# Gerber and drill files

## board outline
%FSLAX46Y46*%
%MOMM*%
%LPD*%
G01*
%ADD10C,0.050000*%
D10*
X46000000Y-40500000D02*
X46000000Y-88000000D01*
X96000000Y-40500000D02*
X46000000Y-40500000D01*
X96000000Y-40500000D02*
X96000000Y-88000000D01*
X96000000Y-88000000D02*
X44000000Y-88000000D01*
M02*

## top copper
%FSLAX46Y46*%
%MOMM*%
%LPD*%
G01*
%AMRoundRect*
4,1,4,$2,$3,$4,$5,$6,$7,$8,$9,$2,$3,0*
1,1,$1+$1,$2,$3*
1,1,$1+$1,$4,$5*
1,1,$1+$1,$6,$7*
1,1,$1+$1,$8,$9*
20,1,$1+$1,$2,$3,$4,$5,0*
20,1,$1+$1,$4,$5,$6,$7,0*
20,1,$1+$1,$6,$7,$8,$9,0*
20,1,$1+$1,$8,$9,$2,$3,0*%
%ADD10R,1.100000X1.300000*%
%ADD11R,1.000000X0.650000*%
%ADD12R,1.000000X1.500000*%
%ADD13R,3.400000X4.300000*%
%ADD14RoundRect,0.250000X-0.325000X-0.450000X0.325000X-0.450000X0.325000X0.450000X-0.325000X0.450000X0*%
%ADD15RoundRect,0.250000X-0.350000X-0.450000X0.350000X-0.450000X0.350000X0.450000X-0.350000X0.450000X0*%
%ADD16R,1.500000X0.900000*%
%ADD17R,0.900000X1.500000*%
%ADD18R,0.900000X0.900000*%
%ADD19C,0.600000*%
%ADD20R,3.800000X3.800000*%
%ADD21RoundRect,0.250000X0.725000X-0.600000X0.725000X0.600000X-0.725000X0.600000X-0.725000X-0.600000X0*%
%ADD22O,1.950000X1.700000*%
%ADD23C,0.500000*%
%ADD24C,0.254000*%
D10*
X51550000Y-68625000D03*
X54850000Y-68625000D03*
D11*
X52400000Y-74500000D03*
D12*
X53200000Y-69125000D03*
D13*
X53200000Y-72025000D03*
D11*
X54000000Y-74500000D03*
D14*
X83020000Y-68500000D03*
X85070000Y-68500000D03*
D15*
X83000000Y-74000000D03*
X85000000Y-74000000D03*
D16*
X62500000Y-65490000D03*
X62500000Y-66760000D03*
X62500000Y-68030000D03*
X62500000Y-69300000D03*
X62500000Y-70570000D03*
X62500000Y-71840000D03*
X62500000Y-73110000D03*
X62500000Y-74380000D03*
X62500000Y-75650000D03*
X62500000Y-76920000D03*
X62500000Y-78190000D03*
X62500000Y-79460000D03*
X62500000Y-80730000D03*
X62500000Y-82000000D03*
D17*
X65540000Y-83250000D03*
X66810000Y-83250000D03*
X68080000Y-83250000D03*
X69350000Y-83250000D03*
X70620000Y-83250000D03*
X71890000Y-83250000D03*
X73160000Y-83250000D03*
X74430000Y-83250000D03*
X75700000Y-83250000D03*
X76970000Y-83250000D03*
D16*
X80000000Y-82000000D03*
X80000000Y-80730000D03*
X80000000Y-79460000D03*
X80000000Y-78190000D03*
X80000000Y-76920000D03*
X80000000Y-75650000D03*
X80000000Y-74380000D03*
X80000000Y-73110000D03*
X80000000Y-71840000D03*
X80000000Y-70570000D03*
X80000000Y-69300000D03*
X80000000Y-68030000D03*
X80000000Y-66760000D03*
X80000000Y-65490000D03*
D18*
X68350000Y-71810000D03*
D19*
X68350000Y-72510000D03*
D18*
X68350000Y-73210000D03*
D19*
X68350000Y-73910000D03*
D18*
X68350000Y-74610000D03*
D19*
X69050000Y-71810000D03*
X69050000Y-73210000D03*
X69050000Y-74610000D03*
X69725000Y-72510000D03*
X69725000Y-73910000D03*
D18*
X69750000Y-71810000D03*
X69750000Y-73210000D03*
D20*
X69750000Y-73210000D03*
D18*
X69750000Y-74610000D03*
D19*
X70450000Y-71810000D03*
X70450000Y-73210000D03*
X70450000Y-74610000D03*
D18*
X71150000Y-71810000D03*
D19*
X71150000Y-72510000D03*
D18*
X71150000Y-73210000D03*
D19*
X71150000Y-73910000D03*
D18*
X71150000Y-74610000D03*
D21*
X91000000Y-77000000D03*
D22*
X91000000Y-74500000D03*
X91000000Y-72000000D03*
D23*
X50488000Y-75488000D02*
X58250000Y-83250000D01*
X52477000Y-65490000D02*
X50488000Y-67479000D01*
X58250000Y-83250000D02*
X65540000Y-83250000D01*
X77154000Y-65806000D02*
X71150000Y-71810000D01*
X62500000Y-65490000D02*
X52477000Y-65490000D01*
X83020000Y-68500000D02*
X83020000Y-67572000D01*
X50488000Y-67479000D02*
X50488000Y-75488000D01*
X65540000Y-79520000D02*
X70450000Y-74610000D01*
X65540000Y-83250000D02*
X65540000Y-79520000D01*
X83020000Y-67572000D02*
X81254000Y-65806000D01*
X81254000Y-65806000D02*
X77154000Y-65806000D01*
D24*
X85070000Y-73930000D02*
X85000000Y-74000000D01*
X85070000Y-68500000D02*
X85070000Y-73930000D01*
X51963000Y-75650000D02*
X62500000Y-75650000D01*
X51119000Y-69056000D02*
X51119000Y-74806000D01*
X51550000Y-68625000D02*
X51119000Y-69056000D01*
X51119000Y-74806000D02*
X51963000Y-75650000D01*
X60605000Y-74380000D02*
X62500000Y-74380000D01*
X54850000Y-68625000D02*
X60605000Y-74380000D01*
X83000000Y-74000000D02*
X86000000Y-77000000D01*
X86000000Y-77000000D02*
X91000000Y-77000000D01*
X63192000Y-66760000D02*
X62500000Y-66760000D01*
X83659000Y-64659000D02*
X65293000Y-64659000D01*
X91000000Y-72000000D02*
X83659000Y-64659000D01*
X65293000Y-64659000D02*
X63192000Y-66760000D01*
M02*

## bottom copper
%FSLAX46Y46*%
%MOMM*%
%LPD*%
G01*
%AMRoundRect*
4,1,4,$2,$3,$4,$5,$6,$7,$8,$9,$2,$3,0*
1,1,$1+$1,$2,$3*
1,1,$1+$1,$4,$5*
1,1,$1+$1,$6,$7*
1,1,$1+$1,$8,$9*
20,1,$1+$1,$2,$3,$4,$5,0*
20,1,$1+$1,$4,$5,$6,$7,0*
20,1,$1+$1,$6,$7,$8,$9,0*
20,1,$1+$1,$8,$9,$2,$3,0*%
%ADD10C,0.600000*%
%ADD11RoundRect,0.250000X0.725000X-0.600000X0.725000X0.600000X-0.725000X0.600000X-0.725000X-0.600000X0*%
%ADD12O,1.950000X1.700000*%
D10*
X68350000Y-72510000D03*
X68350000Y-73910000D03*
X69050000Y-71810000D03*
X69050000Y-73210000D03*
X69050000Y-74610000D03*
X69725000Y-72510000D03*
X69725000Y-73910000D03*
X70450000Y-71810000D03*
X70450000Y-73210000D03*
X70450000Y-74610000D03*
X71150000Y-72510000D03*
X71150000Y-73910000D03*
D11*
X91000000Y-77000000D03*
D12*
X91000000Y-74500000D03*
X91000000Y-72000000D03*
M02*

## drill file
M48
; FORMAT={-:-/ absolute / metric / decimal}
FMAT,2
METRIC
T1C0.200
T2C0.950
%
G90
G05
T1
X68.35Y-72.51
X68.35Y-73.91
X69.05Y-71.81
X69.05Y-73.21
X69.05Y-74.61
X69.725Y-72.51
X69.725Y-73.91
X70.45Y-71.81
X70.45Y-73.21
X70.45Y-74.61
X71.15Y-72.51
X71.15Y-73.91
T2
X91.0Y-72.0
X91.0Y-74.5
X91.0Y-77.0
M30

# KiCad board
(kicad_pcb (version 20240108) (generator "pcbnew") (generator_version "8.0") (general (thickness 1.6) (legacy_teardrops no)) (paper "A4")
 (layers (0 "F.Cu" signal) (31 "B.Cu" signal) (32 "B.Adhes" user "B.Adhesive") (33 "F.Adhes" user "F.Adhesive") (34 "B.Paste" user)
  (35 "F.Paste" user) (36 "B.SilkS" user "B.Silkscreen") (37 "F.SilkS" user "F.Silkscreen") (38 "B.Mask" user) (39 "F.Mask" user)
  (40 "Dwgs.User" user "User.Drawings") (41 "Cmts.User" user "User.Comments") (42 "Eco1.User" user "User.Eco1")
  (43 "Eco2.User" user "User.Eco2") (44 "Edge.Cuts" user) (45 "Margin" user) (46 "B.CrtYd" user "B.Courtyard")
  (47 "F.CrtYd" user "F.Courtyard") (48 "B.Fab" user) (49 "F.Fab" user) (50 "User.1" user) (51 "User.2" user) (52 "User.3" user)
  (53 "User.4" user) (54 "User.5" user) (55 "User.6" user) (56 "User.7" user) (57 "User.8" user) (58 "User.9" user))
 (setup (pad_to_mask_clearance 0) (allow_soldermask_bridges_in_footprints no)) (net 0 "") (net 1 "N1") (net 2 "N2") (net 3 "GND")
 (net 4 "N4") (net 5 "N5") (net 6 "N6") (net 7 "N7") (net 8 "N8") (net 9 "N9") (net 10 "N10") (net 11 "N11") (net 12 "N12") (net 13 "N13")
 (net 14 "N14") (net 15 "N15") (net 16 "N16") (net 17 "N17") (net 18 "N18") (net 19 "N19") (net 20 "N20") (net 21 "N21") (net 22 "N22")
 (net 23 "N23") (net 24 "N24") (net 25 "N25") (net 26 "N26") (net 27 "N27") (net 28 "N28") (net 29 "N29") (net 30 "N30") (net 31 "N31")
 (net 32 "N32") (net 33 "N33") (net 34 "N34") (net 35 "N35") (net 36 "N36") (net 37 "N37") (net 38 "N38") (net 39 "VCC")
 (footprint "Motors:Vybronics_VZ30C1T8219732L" (layer "F.Cu") (at 53.2 72.975)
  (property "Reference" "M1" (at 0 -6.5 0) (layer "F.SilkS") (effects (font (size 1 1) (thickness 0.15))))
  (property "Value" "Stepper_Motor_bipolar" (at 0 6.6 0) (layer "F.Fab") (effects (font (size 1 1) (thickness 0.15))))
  (pad "" smd rect (at -0.85 -2.315 270) (size 1.07 1.4) (layers "F.Paste"))
  (pad "" smd rect (at -0.85 -0.905 270) (size 1.07 1.4) (layers "F.Paste"))
  (pad "" smd rect (at -0.85 0.505 270) (size 1.07 1.4) (layers "F.Paste"))
  (pad "" smd rect (at 0.85 -2.315 270) (size 1.07 1.4) (layers "F.Paste"))
  (pad "" smd rect (at 0.85 -0.905 270) (size 1.07 1.4) (layers "F.Paste"))
  (pad "" smd rect (at 0.85 0.505 270) (size 1.07 1.4) (layers "F.Paste"))
  (pad "1" smd rect (at -1.65 -4.35 270) (size 1.3 1.1) (layers "F.Cu" "F.Paste" "F.Mask") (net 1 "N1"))
  (pad "2" smd rect (at 1.65 -4.35 270) (size 1.3 1.1) (layers "F.Cu" "F.Paste" "F.Mask") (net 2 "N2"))
  (pad "SH" smd rect (at -0.8 1.525) (size 1 0.65) (layers "F.Cu" "F.Paste" "F.Mask"))
  (pad "SH" smd rect (at 0 -3.85 270) (size 1.5 1) (layers "F.Cu" "F.Paste" "F.Mask"))
  (pad "SH" smd rect (at 0 -0.95 270) (size 4.3 3.4) (layers "F.Cu" "F.Mask"))
  (pad "SH" smd rect (at 0.8 1.525) (size 1 0.65) (layers "F.Cu" "F.Paste" "F.Mask")))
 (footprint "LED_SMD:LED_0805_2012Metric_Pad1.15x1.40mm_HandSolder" (layer "F.Cu") (at 84.045 68.5)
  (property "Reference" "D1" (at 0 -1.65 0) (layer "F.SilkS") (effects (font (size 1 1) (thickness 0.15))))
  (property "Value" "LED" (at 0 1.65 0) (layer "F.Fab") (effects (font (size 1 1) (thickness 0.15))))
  (pad "1" smd roundrect (at -1.025 0) (size 1.15 1.4) (layers "F.Cu" "F.Paste" "F.Mask") (roundrect_rratio 0.217391) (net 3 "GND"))
  (pad "2" smd roundrect (at 1.025 0) (size 1.15 1.4) (layers "F.Cu" "F.Paste" "F.Mask") (roundrect_rratio 0.217391) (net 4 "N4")))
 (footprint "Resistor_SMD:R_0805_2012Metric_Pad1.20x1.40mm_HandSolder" (layer "F.Cu") (at 84 74)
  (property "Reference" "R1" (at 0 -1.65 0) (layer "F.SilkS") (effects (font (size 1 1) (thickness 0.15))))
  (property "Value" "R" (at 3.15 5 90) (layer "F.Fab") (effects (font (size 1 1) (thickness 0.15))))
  (pad "1" smd roundrect (at -1 0) (size 1.2 1.4) (layers "F.Cu" "F.Paste" "F.Mask") (roundrect_rratio 0.208333) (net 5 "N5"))
  (pad "2" smd roundrect (at 1 0) (size 1.2 1.4) (layers "F.Cu" "F.Paste" "F.Mask") (roundrect_rratio 0.208333) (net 4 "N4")))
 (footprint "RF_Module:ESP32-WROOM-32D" (layer "F.Cu") (at 71.25 73.74)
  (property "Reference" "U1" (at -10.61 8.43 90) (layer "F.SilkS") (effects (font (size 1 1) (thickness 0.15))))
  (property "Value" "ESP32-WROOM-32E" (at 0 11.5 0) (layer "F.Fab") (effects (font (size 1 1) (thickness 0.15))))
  (pad "1" smd rect (at -8.75 -8.25) (size 1.5 0.9) (layers "F.Cu" "F.Paste" "F.Mask") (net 3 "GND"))
  (pad "2" smd rect (at -8.75 -6.98) (size 1.5 0.9) (layers "F.Cu" "F.Paste" "F.Mask") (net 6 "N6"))
  (pad "3" smd rect (at -8.75 -5.71) (size 1.5 0.9) (layers "F.Cu" "F.Paste" "F.Mask") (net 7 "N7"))
  (pad "4" smd rect (at -8.75 -4.44) (size 1.5 0.9) (layers "F.Cu" "F.Paste" "F.Mask") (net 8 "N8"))
  (pad "5" smd rect (at -8.75 -3.17) (size 1.5 0.9) (layers "F.Cu" "F.Paste" "F.Mask") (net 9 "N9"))
  (pad "6" smd rect (at -8.75 -1.9) (size 1.5 0.9) (layers "F.Cu" "F.Paste" "F.Mask") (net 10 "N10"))
  (pad "7" smd rect (at -8.75 -0.63) (size 1.5 0.9) (layers "F.Cu" "F.Paste" "F.Mask") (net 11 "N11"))
  (pad "8" smd rect (at -8.75 0.64) (size 1.5 0.9) (layers "F.Cu" "F.Paste" "F.Mask") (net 2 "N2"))
  (pad "9" smd rect (at -8.75 1.91) (size 1.5 0.9) (layers "F.Cu" "F.Paste" "F.Mask") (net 1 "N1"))
  (pad "10" smd rect (at -8.75 3.18) (size 1.5 0.9) (layers "F.Cu" "F.Paste" "F.Mask") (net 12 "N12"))
  (pad "11" smd rect (at -8.75 4.45) (size 1.5 0.9) (layers "F.Cu" "F.Paste" "F.Mask") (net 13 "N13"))
  (pad "12" smd rect (at -8.75 5.72) (size 1.5 0.9) (layers "F.Cu" "F.Paste" "F.Mask") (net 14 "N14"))
  (pad "13" smd rect (at -8.75 6.99) (size 1.5 0.9) (layers "F.Cu" "F.Paste" "F.Mask") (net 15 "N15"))
  (pad "14" smd rect (at -8.75 8.26) (size 1.5 0.9) (layers "F.Cu" "F.Paste" "F.Mask") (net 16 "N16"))
  (pad "15" smd rect (at -5.71 9.51 90) (size 1.5 0.9) (layers "F.Cu" "F.Paste" "F.Mask") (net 3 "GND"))
  (pad "16" smd rect (at -4.44 9.51 90) (size 1.5 0.9) (layers "F.Cu" "F.Paste" "F.Mask") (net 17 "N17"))
  (pad "17" smd rect (at -3.17 9.51 90) (size 1.5 0.9) (layers "F.Cu" "F.Paste" "F.Mask") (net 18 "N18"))
  (pad "18" smd rect (at -1.9 9.51 90) (size 1.5 0.9) (layers "F.Cu" "F.Paste" "F.Mask") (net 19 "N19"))
  (pad "19" smd rect (at -0.63 9.51 90) (size 1.5 0.9) (layers "F.Cu" "F.Paste" "F.Mask") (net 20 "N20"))
  (pad "20" smd rect (at 0.64 9.51 90) (size 1.5 0.9) (layers "F.Cu" "F.Paste" "F.Mask") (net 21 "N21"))
  (pad "21" smd rect (at 1.91 9.51 90) (size 1.5 0.9) (layers "F.Cu" "F.Paste" "F.Mask") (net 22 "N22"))
  (pad "22" smd rect (at 3.18 9.51 90) (size 1.5 0.9) (layers "F.Cu" "F.Paste" "F.Mask") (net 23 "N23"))
  (pad "23" smd rect (at 4.45 9.51 90) (size 1.5 0.9) (layers "F.Cu" "F.Paste" "F.Mask") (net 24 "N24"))
  (pad "24" smd rect (at 5.72 9.51 90) (size 1.5 0.9) (layers "F.Cu" "F.Paste" "F.Mask") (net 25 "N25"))
  (pad "25" smd rect (at 8.75 8.26) (size 1.5 0.9) (layers "F.Cu" "F.Paste" "F.Mask") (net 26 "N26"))
  (pad "26" smd rect (at 8.75 6.99) (size 1.5 0.9) (layers "F.Cu" "F.Paste" "F.Mask") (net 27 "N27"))
  (pad "27" smd rect (at 8.75 5.72) (size 1.5 0.9) (layers "F.Cu" "F.Paste" "F.Mask") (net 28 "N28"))
  (pad "28" smd rect (at 8.75 4.45) (size 1.5 0.9) (layers "F.Cu" "F.Paste" "F.Mask") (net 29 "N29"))
  (pad "29" smd rect (at 8.75 3.18) (size 1.5 0.9) (layers "F.Cu" "F.Paste" "F.Mask") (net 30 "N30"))
  (pad "30" smd rect (at 8.75 1.91) (size 1.5 0.9) (layers "F.Cu" "F.Paste" "F.Mask") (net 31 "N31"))
  (pad "31" smd rect (at 8.75 0.64) (size 1.5 0.9) (layers "F.Cu" "F.Paste" "F.Mask") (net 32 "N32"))
  (pad "32" smd rect (at 8.75 -0.63) (size 1.5 0.9) (layers "F.Cu" "F.Paste" "F.Mask") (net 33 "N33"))
  (pad "33" smd rect (at 8.75 -1.9) (size 1.5 0.9) (layers "F.Cu" "F.Paste" "F.Mask") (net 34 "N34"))
  (pad "34" smd rect (at 8.75 -3.17) (size 1.5 0.9) (layers "F.Cu" "F.Paste" "F.Mask") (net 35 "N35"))
  (pad "35" smd rect (at 8.75 -4.44) (size 1.5 0.9) (layers "F.Cu" "F.Paste" "F.Mask") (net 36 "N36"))
  (pad "36" smd rect (at 8.75 -5.71) (size 1.5 0.9) (layers "F.Cu" "F.Paste" "F.Mask") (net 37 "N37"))
  (pad "37" smd rect (at 8.75 -6.98) (size 1.5 0.9) (layers "F.Cu" "F.Paste" "F.Mask") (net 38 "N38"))
  (pad "38" smd rect (at 8.75 -8.25) (size 1.5 0.9) (layers "F.Cu" "F.Paste" "F.Mask") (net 3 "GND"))
  (pad "39" smd rect (at -2.9 -1.93) (size 0.9 0.9) (layers "F.Cu" "F.Paste") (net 3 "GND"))
  (pad "39" thru_hole circle (at -2.9 -1.23) (size 0.6 0.6) (drill 0.2) (layers "*.Cu" "F.Mask") (remove_unused_layers no) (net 3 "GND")
   (zone_connect 2))
  (pad "39" smd rect (at -2.9 -0.53) (size 0.9 0.9) (layers "F.Cu" "F.Paste") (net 3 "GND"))
  (pad "39" thru_hole circle (at -2.9 0.17) (size 0.6 0.6) (drill 0.2) (layers "*.Cu" "F.Mask") (remove_unused_layers no) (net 3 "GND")
   (zone_connect 2))
  (pad "39" smd rect (at -2.9 0.87) (size 0.9 0.9) (layers "F.Cu" "F.Paste") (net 3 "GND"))
  (pad "39" thru_hole circle (at -2.2 -1.93) (size 0.6 0.6) (drill 0.2) (layers "*.Cu" "F.Mask") (remove_unused_layers no) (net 3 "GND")
   (zone_connect 2))
  (pad "39" thru_hole circle (at -2.2 -0.53) (size 0.6 0.6) (drill 0.2) (layers "*.Cu" "F.Mask") (remove_unused_layers no) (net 3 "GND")
   (zone_connect 2))
  (pad "39" thru_hole circle (at -2.2 0.87) (size 0.6 0.6) (drill 0.2) (layers "*.Cu" "F.Mask") (remove_unused_layers no) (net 3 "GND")
   (zone_connect 2))
  (pad "39" thru_hole circle (at -1.525 -1.23) (size 0.6 0.6) (drill 0.2) (layers "*.Cu" "F.Mask") (remove_unused_layers no) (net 3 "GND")
   (zone_connect 2))
  (pad "39" thru_hole circle (at -1.525 0.17) (size 0.6 0.6) (drill 0.2) (layers "*.Cu" "F.Mask") (remove_unused_layers no) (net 3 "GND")
   (zone_connect 2))
  (pad "39" smd rect (at -1.5 -1.93) (size 0.9 0.9) (layers "F.Cu" "F.Paste") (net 3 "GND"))
  (pad "39" smd rect (at -1.5 -0.53) (size 0.9 0.9) (layers "F.Cu" "F.Paste") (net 3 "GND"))
  (pad "39" smd rect (at -1.5 -0.53) (size 3.8 3.8) (layers "F.Cu" "F.Mask") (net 3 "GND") (zone_connect 2))
  (pad "39" smd rect (at -1.5 0.87) (size 0.9 0.9) (layers "F.Cu" "F.Paste") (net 3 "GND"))
  (pad "39" thru_hole circle (at -0.8 -1.93) (size 0.6 0.6) (drill 0.2) (layers "*.Cu" "F.Mask") (remove_unused_layers no) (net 3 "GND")
   (zone_connect 2))
  (pad "39" thru_hole circle (at -0.8 -0.53) (size 0.6 0.6) (drill 0.2) (layers "*.Cu" "F.Mask") (remove_unused_layers no) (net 3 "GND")
   (zone_connect 2))
  (pad "39" thru_hole circle (at -0.8 0.87) (size 0.6 0.6) (drill 0.2) (layers "*.Cu" "F.Mask") (remove_unused_layers no) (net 3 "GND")
   (zone_connect 2))
  (pad "39" smd rect (at -0.1 -1.93) (size 0.9 0.9) (layers "F.Cu" "F.Paste") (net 3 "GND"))
  (pad "39" thru_hole circle (at -0.1 -1.23) (size 0.6 0.6) (drill 0.2) (layers "*.Cu" "F.Mask") (remove_unused_layers no) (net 3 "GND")
   (zone_connect 2))
  (pad "39" smd rect (at -0.1 -0.53) (size 0.9 0.9) (layers "F.Cu" "F.Paste") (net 3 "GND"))
  (pad "39" thru_hole circle (at -0.1 0.17) (size 0.6 0.6) (drill 0.2) (layers "*.Cu" "F.Mask") (remove_unused_layers no) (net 3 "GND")
   (zone_connect 2))
  (pad "39" smd rect (at -0.1 0.87) (size 0.9 0.9) (layers "F.Cu" "F.Paste") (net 3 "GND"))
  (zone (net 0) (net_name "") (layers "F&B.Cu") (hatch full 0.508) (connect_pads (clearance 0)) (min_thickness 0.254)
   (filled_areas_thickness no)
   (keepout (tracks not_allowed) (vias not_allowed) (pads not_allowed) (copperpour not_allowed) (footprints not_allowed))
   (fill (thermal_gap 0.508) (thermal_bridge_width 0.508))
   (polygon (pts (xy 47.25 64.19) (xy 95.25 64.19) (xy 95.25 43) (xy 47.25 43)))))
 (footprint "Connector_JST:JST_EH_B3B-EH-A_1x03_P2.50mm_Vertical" (layer "F.Cu") (at 91 77 90)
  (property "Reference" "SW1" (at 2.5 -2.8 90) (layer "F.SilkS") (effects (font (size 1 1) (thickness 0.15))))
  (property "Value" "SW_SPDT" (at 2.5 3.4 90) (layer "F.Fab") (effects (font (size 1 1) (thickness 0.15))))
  (pad "1" thru_hole roundrect (at 0 0 90) (size 1.7 1.95) (drill 0.95) (layers "*.Cu" "*.Mask") (remove_unused_layers no)
   (roundrect_rratio 0.147059) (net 5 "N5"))
  (pad "2" thru_hole oval (at 2.5 0 90) (size 1.7 1.95) (drill 0.95) (layers "*.Cu" "*.Mask") (remove_unused_layers no) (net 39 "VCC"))
  (pad "3" thru_hole oval (at 5 0 90) (size 1.7 1.95) (drill 0.95) (layers "*.Cu" "*.Mask") (remove_unused_layers no) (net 6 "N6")))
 (gr_line (start 46 40.5) (end 46 88) (stroke (width 0.05) (type default)) (layer "Edge.Cuts"))
 (gr_line (start 96 40.5) (end 46 40.5) (stroke (width 0.05) (type default)) (layer "Edge.Cuts"))
 (gr_line (start 96 40.5) (end 96 88) (stroke (width 0.05) (type default)) (layer "Edge.Cuts"))
 (gr_line (start 96 88) (end 44 88) (stroke (width 0.05) (type default)) (layer "Edge.Cuts"))
 (segment (start 50.488 75.488) (end 58.25 83.25) (width 0.5) (layer "F.Cu") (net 3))
 (segment (start 52.477 65.49) (end 50.488 67.479) (width 0.5) (layer "F.Cu") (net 3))
 (segment (start 58.25 83.25) (end 65.54 83.25) (width 0.5) (layer "F.Cu") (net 3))
 (segment (start 77.154 65.806) (end 71.15 71.81) (width 0.5) (layer "F.Cu") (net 3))
 (segment (start 62.5 65.49) (end 52.477 65.49) (width 0.5) (layer "F.Cu") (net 3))
 (segment (start 83.02 68.5) (end 83.02 67.572) (width 0.5) (layer "F.Cu") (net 3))
 (segment (start 50.488 67.479) (end 50.488 75.488) (width 0.5) (layer "F.Cu") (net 3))
 (segment (start 65.54 79.52) (end 70.45 74.61) (width 0.5) (layer "F.Cu") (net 3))
 (segment (start 65.54 83.25) (end 65.54 79.52) (width 0.5) (layer "F.Cu") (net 3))
 (segment (start 83.02 67.572) (end 81.254 65.806) (width 0.5) (layer "F.Cu") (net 3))
 (segment (start 81.254 65.806) (end 77.154 65.806) (width 0.5) (layer "F.Cu") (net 3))
 (segment (start 85.07 73.93) (end 85 74) (width 0.254) (layer "F.Cu") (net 4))
 (segment (start 85.07 68.5) (end 85.07 73.93) (width 0.254) (layer "F.Cu") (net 4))
 (segment (start 51.963 75.65) (end 62.5 75.65) (width 0.254) (layer "F.Cu") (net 1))
 (segment (start 51.119 69.056) (end 51.119 74.806) (width 0.254) (layer "F.Cu") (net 1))
 (segment (start 51.55 68.625) (end 51.119 69.056) (width 0.254) (layer "F.Cu") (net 1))
 (segment (start 51.119 74.806) (end 51.963 75.65) (width 0.254) (layer "F.Cu") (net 1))
 (segment (start 60.605 74.38) (end 62.5 74.38) (width 0.254) (layer "F.Cu") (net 2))
 (segment (start 54.85 68.625) (end 60.605 74.38) (width 0.254) (layer "F.Cu") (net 2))
 (segment (start 83 74) (end 86 77) (width 0.254) (layer "F.Cu") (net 5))
 (segment (start 86 77) (end 91 77) (width 0.254) (layer "F.Cu") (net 5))
 (segment (start 63.192 66.76) (end 62.5 66.76) (width 0.254) (layer "F.Cu") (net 6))
 (segment (start 83.659 64.659) (end 65.293 64.659) (width 0.254) (layer "F.Cu") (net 6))
 (segment (start 91 72) (end 83.659 64.659) (width 0.254) (layer "F.Cu") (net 6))
 (segment (start 65.293 64.659) (end 63.192 66.76) (width 0.254) (layer "F.Cu") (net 6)))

